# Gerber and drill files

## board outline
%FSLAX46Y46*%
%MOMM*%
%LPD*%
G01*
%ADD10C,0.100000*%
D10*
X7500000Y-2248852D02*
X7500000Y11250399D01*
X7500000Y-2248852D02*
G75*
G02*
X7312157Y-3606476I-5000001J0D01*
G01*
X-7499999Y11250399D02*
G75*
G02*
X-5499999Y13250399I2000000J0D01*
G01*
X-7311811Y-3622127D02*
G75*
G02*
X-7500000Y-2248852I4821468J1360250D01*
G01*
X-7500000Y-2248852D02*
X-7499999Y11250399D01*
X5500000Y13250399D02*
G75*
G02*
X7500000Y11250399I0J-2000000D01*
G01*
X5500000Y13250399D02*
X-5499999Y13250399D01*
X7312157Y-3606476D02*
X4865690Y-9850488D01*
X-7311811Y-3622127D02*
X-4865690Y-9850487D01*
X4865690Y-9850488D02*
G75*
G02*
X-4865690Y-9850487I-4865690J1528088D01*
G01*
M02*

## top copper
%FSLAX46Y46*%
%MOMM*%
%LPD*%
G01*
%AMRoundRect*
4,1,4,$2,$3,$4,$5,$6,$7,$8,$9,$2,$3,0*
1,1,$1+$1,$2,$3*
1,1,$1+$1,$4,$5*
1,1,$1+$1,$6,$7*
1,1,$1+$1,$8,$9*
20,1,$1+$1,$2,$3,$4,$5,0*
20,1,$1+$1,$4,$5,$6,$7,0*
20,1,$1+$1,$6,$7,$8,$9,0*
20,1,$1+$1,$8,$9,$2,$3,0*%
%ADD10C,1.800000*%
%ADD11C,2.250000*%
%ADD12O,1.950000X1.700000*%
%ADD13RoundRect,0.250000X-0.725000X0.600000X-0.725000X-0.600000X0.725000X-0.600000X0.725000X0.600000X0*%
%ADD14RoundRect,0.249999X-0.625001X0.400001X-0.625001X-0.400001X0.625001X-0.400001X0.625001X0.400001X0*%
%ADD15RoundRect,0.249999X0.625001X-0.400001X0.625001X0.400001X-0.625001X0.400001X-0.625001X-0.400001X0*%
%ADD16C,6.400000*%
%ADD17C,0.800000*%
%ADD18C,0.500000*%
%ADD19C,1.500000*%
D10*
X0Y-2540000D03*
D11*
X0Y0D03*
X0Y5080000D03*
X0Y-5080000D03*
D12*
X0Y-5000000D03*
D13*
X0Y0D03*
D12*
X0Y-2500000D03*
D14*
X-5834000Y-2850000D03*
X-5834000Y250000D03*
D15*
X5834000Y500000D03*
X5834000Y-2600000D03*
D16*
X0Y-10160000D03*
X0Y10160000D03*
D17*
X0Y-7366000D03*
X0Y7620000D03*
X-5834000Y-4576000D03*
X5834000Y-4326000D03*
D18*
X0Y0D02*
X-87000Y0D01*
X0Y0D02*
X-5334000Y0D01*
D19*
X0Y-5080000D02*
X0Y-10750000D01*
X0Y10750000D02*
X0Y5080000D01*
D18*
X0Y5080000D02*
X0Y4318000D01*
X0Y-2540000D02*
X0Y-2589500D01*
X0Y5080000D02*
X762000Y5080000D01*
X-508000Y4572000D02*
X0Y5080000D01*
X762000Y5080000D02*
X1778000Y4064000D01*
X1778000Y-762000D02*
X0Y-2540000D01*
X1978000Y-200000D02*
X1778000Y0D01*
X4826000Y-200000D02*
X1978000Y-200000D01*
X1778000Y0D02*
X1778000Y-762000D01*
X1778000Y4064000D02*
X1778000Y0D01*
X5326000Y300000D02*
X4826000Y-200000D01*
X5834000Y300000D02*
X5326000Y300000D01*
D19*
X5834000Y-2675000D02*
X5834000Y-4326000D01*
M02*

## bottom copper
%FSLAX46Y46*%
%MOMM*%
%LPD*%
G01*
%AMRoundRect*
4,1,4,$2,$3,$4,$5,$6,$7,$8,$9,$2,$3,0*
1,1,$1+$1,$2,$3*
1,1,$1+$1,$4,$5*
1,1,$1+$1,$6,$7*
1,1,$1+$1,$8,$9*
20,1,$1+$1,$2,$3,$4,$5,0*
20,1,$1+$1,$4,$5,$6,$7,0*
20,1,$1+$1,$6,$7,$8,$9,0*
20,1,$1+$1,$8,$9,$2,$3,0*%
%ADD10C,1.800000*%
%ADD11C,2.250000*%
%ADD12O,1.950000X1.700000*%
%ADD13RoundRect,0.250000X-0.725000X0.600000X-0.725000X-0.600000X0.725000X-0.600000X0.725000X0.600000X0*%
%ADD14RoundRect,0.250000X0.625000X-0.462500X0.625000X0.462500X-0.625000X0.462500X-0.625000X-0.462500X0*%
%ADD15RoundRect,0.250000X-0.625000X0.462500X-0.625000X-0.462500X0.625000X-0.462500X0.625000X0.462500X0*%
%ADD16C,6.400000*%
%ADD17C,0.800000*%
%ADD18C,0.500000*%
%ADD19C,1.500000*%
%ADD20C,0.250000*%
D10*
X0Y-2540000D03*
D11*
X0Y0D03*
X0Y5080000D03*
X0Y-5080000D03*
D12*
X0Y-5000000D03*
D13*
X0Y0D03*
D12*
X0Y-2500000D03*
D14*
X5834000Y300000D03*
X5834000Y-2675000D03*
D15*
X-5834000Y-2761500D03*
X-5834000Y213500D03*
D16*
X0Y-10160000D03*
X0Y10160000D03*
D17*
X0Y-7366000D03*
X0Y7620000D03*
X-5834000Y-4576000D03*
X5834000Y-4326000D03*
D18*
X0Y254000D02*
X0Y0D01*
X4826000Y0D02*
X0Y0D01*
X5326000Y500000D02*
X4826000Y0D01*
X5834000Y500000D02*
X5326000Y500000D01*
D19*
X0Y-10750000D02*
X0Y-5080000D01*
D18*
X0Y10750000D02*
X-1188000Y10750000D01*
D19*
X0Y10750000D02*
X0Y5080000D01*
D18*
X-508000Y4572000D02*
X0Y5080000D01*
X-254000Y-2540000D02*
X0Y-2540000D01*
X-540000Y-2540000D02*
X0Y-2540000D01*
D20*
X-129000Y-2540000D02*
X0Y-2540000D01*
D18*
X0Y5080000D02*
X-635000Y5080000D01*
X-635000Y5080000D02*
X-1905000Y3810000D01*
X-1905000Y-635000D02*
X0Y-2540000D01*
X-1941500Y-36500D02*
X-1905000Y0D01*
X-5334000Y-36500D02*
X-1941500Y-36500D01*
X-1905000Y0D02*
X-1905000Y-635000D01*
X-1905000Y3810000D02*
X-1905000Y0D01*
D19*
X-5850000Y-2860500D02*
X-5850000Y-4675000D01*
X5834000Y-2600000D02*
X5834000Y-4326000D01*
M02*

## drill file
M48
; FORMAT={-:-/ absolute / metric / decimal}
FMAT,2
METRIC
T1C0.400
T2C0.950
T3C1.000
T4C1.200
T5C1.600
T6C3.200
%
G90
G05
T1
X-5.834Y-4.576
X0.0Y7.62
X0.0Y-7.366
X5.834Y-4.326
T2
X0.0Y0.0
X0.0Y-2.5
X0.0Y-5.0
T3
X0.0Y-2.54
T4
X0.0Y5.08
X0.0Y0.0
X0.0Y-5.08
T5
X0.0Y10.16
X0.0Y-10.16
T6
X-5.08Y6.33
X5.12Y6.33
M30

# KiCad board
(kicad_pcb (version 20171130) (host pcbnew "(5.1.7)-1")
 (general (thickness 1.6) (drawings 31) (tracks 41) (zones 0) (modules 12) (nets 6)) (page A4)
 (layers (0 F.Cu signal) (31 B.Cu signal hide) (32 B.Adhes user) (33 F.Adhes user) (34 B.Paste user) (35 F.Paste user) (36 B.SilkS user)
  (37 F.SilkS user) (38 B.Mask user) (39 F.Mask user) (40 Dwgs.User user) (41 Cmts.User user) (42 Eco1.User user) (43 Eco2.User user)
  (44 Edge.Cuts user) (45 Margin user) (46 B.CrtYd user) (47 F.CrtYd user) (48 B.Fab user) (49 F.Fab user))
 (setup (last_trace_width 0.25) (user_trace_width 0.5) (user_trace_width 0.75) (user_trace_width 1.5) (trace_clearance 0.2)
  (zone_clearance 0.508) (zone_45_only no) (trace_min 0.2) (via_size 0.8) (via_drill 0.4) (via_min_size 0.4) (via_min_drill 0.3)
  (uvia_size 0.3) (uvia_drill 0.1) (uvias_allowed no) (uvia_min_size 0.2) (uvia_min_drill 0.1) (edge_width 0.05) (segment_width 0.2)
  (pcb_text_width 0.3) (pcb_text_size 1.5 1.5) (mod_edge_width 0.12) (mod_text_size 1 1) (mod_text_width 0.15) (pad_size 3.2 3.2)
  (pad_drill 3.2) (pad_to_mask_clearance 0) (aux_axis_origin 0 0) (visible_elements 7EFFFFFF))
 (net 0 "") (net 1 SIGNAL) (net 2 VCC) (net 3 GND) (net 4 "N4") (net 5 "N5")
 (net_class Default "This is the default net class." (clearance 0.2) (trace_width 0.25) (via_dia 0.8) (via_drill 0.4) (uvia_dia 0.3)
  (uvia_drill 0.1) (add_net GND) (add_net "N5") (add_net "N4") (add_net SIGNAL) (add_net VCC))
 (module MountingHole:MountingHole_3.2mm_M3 (layer F.Cu) (at -5.08 -6.33)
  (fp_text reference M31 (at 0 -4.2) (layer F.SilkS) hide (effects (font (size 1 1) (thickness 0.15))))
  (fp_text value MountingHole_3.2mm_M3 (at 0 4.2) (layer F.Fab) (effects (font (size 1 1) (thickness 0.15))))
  (pad "" np_thru_hole circle (at 0 0) (size 3.2 3.2) (drill 3.2) (layers *.Cu *.Mask)))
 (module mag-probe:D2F (layer F.Cu) (at 0 0 270)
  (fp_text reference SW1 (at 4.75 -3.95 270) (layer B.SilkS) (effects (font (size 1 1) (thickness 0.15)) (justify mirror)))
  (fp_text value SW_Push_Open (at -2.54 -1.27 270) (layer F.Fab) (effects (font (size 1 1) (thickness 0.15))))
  (pad 4 thru_hole circle (at 2.54 0 270) (size 1.8 1.8) (drill 1) (layers *.Cu *.Mask) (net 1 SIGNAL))
  (pad 3 thru_hole circle (at 0 0 270) (size 2.25 2.25) (drill 1.2) (layers *.Cu *.Mask) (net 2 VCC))
  (pad 2 thru_hole circle (at -5.08 0 270) (size 2.25 2.25) (drill 1.2) (layers *.Cu *.Mask) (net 1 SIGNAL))
  (pad 1 thru_hole circle (at 5.08 0 270) (size 2.25 2.25) (drill 1.2) (layers *.Cu *.Mask) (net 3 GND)))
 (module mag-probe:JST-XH (layer F.Cu) (at 0 0 270)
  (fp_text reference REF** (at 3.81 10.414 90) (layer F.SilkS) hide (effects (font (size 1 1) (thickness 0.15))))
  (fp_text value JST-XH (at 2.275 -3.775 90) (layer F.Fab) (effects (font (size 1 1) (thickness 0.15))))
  (pad 3 thru_hole oval (at 5 0 270) (size 1.7 1.95) (drill 0.95) (layers *.Cu *.Mask))
  (pad 1 thru_hole roundrect (at 0 0 270) (size 1.7 1.95) (drill 0.95) (layers *.Cu *.Mask) (roundrect_rratio 0.1470588235294118))
  (pad 2 thru_hole oval (at 2.5 0 270) (size 1.7 1.95) (drill 0.95) (layers *.Cu *.Mask)))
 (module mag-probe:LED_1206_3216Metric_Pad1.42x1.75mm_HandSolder (layer B.Cu) (at 5.834 1.1875 90)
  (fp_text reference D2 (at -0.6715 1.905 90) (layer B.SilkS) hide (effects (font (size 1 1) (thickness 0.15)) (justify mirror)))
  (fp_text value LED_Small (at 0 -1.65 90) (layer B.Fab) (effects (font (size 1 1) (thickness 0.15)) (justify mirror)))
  (pad 2 smd roundrect (at 1.4875 0 90) (size 1.425 1.75) (layers B.Cu B.Paste B.Mask) (roundrect_rratio 0.1754385964912281) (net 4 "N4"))
  (pad 1 smd roundrect (at -1.4875 0 90) (size 1.425 1.75) (layers B.Cu B.Paste B.Mask) (roundrect_rratio 0.1754385964912281) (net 1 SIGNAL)))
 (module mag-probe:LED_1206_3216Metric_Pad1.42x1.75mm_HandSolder (layer B.Cu) (at -5.834 1.274 270)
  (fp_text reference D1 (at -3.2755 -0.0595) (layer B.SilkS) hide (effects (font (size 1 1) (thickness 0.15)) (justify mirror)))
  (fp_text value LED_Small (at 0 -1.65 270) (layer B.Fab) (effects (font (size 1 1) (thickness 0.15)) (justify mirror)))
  (pad 2 smd roundrect (at 1.4875 0 270) (size 1.425 1.75) (layers B.Cu B.Paste B.Mask) (roundrect_rratio 0.1754385964912281) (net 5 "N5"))
  (pad 1 smd roundrect (at -1.4875 0 270) (size 1.425 1.75) (layers B.Cu B.Paste B.Mask) (roundrect_rratio 0.1754385964912281)
   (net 1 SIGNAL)))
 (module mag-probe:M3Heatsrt (layer F.Cu) (at -5.08 -6.33)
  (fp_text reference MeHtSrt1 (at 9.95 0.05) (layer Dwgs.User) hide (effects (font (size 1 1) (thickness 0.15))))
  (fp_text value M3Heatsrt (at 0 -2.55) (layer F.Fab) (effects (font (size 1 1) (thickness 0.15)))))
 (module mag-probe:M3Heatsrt (layer F.Cu) (at 5.08 -6.33)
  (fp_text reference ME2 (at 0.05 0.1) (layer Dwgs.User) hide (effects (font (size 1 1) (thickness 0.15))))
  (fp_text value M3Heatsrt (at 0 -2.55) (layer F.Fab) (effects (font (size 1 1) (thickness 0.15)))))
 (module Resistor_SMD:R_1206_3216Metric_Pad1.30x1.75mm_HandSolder (layer F.Cu) (at -5.834 1.3 270)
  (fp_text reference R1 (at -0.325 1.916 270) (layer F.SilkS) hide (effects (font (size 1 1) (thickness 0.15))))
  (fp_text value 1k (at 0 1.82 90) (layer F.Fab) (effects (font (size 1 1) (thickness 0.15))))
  (pad 2 smd roundrect (at 1.55 0 270) (size 1.3 1.75) (layers F.Cu F.Paste F.Mask) (roundrect_rratio 0.1923069230769231) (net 5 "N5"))
  (pad 1 smd roundrect (at -1.55 0 270) (size 1.3 1.75) (layers F.Cu F.Paste F.Mask) (roundrect_rratio 0.1923069230769231) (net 2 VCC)))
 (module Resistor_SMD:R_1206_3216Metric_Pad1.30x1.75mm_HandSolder (layer F.Cu) (at 5.834 1.05 90)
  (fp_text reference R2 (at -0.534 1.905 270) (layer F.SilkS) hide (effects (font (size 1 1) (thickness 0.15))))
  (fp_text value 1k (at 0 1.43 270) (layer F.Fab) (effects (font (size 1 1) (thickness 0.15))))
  (pad 2 smd roundrect (at 1.55 0 90) (size 1.3 1.75) (layers F.Cu F.Paste F.Mask) (roundrect_rratio 0.1923069230769231) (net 4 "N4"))
  (pad 1 smd roundrect (at -1.55 0 90) (size 1.3 1.75) (layers F.Cu F.Paste F.Mask) (roundrect_rratio 0.1923069230769231) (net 2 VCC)))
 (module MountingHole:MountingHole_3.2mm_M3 (layer F.Cu) (at 5.08 -6.33)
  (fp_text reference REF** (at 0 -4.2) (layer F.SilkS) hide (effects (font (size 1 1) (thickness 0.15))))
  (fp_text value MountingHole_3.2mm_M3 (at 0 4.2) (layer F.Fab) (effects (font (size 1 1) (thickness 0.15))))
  (pad "" np_thru_hole circle (at 0.04 0) (size 3.2 3.2) (drill 3.2) (layers *.Cu *.Mask)))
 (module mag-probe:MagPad (layer B.Cu) (at 0 10.16)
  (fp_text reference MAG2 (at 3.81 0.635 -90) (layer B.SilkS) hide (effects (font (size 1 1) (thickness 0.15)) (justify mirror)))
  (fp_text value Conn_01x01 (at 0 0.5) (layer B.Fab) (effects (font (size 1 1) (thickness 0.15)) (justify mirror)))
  (pad 1 thru_hole circle (at 0 0) (size 6.4 6.4) (drill 1.6) (layers *.Cu *.Mask) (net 3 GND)))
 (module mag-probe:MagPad (layer B.Cu) (at 0 -10.16)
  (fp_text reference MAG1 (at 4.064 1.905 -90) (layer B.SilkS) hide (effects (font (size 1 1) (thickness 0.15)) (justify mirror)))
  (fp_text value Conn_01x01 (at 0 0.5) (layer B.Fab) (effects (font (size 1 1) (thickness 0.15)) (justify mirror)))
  (pad 1 thru_hole circle (at 0 0) (size 6.4 6.4) (drill 1.6) (layers *.Cu *.Mask) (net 1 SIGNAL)))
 (gr_line (start 7.5 2.248852) (end 7.5 -11.250399) (layer Edge.Cuts) (width 0.1))
 (gr_arc (start 2.499999 2.248852) (end 7.312157 3.606476) (angle -15.75501346) (layer Edge.Cuts) (width 0.1))
 (gr_arc (start -5.499999 -11.250399) (end -5.499999 -13.250399) (angle -90) (layer Edge.Cuts) (width 0.1))
 (gr_arc (start -2.490343 2.261877) (end -7.5 2.248852) (angle -15.90398022) (layer Edge.Cuts) (width 0.1))
 (gr_line (start -7.5 2.248852) (end -7.499999 -11.250399) (layer Edge.Cuts) (width 0.1))
 (gr_arc (start 5.5 -11.250399) (end 7.5 -11.250399) (angle -90) (layer Edge.Cuts) (width 0.1))
 (gr_line (start 5.5 -13.250399) (end -5.499999 -13.250399) (layer Edge.Cuts) (width 0.1))
 (gr_line (start 7.312157 3.606476) (end 4.86569 9.850488) (layer Edge.Cuts) (width 0.1))
 (gr_line (start -7.311811 3.622127) (end -4.86569 9.850487) (layer Edge.Cuts) (width 0.1))
 (gr_arc (start 0 8.3224) (end -4.86569 9.850487) (angle -145.1298326) (layer Edge.Cuts) (width 0.1))
 (segment (start 0 -0.254) (end 0 0) (width 0.5) (layer B.Cu) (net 2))
 (segment (start 0 0) (end -0.087 0) (width 0.5) (layer F.Cu) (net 2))
 (segment (start 4.826 0) (end 0 0) (width 0.5) (layer B.Cu) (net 2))
 (segment (start 0 0) (end -5.334 0) (width 0.5) (layer F.Cu) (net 2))
 (segment (start 5.326 -0.5) (end 4.826 0) (width 0.5) (layer B.Cu) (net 2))
 (segment (start 5.834 -0.5) (end 5.326 -0.5) (width 0.5) (layer B.Cu) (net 2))
 (segment (start 0 10.75) (end 0 5.08) (width 1.5) (layer B.Cu) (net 3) (status 30))
 (segment (start 0 5.08) (end 0 10.75) (width 1.5) (layer F.Cu) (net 3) (status 30))
 (via (at 0 7.366) (size 0.8) (drill 0.4) (layers F.Cu B.Cu) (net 3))
 (via (at 0 -7.62) (size 0.8) (drill 0.4) (layers F.Cu B.Cu) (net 1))
 (segment (start 0 -10.75) (end -1.188 -10.75) (width 0.5) (layer B.Cu) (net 1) (status 30))
 (segment (start 0 -10.75) (end 0 -5.08) (width 1.5) (layer B.Cu) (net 1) (status 30))
 (segment (start -0.508 -4.572) (end 0 -5.08) (width 0.5) (layer B.Cu) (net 1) (status 30))
 (segment (start 0 -10.75) (end 0 -5.08) (width 1.5) (layer F.Cu) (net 1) (status 30))
 (segment (start -0.254 2.54) (end 0 2.54) (width 0.5) (layer B.Cu) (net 1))
 (segment (start 0 -5.08) (end 0 -4.318) (width 0.5) (layer F.Cu) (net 1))
 (segment (start 0 2.54) (end 0 2.5895) (width 0.5) (layer F.Cu) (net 1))
 (segment (start -0.54 2.54) (end 0 2.54) (width 0.5) (layer B.Cu) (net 1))
 (segment (start -0.129 2.54) (end 0 2.54) (width 0.25) (layer B.Cu) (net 1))
 (segment (start 0 -5.08) (end 0.762 -5.08) (width 0.5) (layer F.Cu) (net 1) (status 30))
 (segment (start -0.508 -4.572) (end 0 -5.08) (width 0.5) (layer F.Cu) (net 1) (status 30))
 (segment (start 0 -5.08) (end -0.635 -5.08) (width 0.5) (layer B.Cu) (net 1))
 (segment (start -0.635 -5.08) (end -1.905 -3.81) (width 0.5) (layer B.Cu) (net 1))
 (segment (start -1.905 0.635) (end 0 2.54) (width 0.5) (layer B.Cu) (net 1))
 (segment (start 0.762 -5.08) (end 1.778 -4.064) (width 0.5) (layer F.Cu) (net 1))
 (segment (start 1.778 0.762) (end 0 2.54) (width 0.5) (layer F.Cu) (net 1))
 (segment (start 1.978 0.2) (end 1.778 0) (width 0.5) (layer F.Cu) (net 1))
 (segment (start 4.826 0.2) (end 1.978 0.2) (width 0.5) (layer F.Cu) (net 1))
 (segment (start 1.778 0) (end 1.778 0.762) (width 0.5) (layer F.Cu) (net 1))
 (segment (start 1.778 -4.064) (end 1.778 0) (width 0.5) (layer F.Cu) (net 1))
 (segment (start -1.9415 0.0365) (end -1.905 0) (width 0.5) (layer B.Cu) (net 1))
 (segment (start -5.334 0.0365) (end -1.9415 0.0365) (width 0.5) (layer B.Cu) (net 1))
 (segment (start -1.905 0) (end -1.905 0.635) (width 0.5) (layer B.Cu) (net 1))
 (segment (start -1.905 -3.81) (end -1.905 0) (width 0.5) (layer B.Cu) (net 1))
 (segment (start 5.326 -0.3) (end 4.826 0.2) (width 0.5) (layer F.Cu) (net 1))
 (segment (start 5.834 -0.3) (end 5.326 -0.3) (width 0.5) (layer F.Cu) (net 1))
 (via (at -5.834 4.576) (size 0.8) (drill 0.4) (layers F.Cu B.Cu) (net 5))
 (segment (start -5.85 2.8605) (end -5.85 4.675) (width 1.5) (layer B.Cu) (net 5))
 (via (at 5.834 4.326) (size 0.8) (drill 0.4) (layers F.Cu B.Cu) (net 4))
 (segment (start 5.834 2.6) (end 5.834 4.326) (width 1.5) (layer B.Cu) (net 4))
 (segment (start 5.834 2.675) (end 5.834 4.326) (width 1.5) (layer F.Cu) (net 4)))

